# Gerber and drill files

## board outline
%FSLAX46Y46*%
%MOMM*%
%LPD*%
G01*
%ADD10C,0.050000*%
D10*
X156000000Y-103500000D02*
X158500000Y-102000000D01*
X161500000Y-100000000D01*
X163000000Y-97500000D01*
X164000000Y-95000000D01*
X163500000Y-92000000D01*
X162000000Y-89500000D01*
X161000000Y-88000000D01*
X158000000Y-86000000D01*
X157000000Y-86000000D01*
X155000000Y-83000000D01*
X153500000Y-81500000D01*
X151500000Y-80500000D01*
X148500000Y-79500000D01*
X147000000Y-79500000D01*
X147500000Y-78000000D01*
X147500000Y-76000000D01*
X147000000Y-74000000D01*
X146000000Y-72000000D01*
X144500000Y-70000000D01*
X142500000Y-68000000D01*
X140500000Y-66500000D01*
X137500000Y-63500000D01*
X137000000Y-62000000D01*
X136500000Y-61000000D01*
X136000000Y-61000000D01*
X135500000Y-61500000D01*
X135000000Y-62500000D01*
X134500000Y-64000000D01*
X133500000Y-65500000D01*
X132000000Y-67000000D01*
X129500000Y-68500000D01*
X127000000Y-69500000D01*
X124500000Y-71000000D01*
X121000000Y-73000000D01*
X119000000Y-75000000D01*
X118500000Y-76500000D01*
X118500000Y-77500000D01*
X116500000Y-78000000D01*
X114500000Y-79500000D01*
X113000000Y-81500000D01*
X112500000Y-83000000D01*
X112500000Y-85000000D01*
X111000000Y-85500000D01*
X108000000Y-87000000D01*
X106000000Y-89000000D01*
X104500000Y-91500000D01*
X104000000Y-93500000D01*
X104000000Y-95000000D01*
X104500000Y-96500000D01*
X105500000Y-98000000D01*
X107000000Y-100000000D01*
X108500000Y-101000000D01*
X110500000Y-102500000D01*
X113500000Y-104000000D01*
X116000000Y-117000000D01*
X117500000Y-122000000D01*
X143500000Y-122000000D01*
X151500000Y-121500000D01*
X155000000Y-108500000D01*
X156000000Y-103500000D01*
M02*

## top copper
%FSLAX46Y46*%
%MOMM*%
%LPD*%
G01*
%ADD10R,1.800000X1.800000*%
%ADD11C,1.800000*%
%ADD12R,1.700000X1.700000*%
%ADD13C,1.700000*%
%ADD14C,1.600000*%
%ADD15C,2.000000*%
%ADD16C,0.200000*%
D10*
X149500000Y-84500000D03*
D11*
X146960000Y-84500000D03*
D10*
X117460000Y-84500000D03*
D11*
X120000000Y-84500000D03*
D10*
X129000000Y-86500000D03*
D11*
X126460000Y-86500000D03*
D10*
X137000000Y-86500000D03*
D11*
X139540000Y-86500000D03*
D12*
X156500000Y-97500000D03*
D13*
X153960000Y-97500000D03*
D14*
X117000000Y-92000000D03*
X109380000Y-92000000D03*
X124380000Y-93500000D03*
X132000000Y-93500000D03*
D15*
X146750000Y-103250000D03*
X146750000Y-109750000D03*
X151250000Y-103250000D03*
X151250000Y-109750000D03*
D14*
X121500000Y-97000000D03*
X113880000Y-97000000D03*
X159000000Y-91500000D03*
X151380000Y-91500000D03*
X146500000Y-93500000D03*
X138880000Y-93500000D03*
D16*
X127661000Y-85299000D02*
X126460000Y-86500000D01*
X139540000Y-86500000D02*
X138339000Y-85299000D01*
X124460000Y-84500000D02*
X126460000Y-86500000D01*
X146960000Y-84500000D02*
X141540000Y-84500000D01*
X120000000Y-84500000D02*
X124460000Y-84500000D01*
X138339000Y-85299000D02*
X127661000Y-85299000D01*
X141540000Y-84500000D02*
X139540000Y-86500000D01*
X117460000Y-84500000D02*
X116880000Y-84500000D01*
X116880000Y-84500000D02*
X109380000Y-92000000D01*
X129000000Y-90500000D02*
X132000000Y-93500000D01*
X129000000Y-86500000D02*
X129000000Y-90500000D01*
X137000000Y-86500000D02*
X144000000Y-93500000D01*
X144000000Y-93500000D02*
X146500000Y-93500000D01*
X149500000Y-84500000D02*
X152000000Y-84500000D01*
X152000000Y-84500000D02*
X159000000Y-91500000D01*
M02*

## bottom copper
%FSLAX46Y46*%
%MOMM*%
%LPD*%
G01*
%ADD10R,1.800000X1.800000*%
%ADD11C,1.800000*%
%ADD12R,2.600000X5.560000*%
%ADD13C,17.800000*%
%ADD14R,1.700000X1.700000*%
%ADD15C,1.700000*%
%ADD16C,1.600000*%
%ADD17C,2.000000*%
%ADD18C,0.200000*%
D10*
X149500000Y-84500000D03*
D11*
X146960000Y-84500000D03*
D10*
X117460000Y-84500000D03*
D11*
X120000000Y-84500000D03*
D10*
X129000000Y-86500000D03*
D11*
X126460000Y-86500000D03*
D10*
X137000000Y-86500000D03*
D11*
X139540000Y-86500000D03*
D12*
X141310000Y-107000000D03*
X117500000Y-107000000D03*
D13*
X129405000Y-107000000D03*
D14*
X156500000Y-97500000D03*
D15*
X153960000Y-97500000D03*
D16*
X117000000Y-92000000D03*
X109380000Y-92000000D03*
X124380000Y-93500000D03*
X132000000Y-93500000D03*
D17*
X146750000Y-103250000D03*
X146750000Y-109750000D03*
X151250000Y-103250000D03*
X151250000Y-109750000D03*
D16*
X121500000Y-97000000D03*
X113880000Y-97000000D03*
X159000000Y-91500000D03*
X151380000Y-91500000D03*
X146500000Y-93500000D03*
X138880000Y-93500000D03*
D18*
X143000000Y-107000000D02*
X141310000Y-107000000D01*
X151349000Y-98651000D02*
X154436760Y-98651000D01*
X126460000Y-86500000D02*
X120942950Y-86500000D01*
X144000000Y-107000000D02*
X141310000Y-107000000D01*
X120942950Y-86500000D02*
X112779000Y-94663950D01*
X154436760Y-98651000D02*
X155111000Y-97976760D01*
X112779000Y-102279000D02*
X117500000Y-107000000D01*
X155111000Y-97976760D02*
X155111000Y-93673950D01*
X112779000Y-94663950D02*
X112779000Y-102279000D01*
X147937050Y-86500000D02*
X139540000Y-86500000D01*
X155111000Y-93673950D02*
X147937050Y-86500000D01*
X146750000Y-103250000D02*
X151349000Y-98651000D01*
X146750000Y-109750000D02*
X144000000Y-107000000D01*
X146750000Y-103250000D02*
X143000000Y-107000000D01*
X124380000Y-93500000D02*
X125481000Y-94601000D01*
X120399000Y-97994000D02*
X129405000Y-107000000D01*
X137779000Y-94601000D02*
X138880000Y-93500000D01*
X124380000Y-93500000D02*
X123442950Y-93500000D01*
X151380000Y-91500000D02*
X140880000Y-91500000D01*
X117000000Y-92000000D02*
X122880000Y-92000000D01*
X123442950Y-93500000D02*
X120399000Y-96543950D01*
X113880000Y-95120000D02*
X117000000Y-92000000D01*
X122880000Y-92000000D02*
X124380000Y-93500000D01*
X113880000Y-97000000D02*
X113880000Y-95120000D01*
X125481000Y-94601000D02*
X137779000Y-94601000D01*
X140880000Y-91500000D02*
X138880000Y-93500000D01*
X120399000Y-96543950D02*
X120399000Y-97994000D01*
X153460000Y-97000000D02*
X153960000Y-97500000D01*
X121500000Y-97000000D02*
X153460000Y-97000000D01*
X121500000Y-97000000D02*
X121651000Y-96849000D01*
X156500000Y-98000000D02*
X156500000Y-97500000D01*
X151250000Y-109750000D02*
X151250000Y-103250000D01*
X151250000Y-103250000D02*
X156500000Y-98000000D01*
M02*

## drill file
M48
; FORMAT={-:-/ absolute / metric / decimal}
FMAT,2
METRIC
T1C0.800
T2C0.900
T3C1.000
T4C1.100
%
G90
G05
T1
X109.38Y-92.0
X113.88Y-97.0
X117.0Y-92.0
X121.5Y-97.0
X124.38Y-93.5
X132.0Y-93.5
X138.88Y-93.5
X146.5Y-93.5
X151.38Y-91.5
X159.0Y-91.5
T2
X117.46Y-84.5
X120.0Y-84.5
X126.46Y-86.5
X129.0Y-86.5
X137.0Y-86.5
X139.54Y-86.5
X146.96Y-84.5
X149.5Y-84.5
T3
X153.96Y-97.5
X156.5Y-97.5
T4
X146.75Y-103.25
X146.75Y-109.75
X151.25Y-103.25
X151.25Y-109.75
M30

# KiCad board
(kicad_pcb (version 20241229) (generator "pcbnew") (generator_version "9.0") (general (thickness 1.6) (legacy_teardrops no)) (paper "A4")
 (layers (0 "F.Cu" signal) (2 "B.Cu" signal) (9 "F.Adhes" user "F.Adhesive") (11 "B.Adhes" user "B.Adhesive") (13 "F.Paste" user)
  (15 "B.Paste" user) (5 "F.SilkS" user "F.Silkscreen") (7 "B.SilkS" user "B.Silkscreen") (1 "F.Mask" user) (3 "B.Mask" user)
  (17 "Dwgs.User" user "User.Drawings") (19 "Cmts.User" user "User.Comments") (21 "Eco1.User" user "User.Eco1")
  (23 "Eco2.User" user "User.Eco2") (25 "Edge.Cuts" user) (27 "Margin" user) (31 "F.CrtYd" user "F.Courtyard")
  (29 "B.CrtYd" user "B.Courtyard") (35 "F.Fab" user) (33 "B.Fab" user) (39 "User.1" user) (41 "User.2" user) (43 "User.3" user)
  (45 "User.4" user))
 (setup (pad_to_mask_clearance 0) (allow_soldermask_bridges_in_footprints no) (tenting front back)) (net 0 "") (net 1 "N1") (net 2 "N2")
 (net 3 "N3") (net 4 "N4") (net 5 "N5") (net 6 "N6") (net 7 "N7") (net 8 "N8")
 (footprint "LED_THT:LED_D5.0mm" (layer "F.Cu") (at 149.5 84.5 180)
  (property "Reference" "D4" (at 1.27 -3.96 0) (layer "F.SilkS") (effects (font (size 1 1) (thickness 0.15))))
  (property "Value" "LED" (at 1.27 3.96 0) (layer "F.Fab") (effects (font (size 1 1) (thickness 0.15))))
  (pad "1" thru_hole rect (at 0 0 180) (size 1.8 1.8) (drill 0.9) (layers "*.Cu" "*.Mask") (remove_unused_layers no) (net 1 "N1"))
  (pad "2" thru_hole circle (at 2.54 0 180) (size 1.8 1.8) (drill 0.9) (layers "*.Cu" "*.Mask") (remove_unused_layers no) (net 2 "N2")))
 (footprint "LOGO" (layer "F.Cu") (at 134.5 112)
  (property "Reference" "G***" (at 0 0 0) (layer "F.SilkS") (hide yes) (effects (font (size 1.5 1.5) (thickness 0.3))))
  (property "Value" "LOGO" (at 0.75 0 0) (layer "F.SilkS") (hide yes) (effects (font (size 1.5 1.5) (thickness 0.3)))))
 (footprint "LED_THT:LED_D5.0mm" (layer "F.Cu") (at 117.46 84.5)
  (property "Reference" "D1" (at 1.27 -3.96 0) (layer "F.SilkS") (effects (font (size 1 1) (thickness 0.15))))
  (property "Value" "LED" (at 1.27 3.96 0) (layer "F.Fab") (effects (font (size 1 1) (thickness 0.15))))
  (pad "1" thru_hole rect (at 0 0) (size 1.8 1.8) (drill 0.9) (layers "*.Cu" "*.Mask") (remove_unused_layers no) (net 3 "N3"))
  (pad "2" thru_hole circle (at 2.54 0) (size 1.8 1.8) (drill 0.9) (layers "*.Cu" "*.Mask") (remove_unused_layers no) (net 2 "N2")))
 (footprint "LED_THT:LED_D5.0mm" (layer "F.Cu") (at 129 86.5 180)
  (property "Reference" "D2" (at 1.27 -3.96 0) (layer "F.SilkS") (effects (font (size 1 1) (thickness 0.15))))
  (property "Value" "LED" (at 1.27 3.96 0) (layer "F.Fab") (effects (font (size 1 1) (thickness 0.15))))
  (pad "1" thru_hole rect (at 0 0 180) (size 1.8 1.8) (drill 0.9) (layers "*.Cu" "*.Mask") (remove_unused_layers no) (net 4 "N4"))
  (pad "2" thru_hole circle (at 2.54 0 180) (size 1.8 1.8) (drill 0.9) (layers "*.Cu" "*.Mask") (remove_unused_layers no) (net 2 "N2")))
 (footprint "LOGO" (layer "F.Cu") (at 133 73.5)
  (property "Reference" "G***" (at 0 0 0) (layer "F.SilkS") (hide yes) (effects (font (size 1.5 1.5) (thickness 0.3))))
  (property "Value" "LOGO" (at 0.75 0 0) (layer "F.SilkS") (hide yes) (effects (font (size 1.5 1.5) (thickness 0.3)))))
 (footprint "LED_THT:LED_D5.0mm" (layer "F.Cu") (at 137 86.5)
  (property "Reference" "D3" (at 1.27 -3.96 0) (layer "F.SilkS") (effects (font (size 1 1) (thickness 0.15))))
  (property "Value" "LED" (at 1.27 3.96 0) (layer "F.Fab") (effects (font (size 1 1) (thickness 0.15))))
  (pad "1" thru_hole rect (at 0 0) (size 1.8 1.8) (drill 0.9) (layers "*.Cu" "*.Mask") (remove_unused_layers no) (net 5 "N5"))
  (pad "2" thru_hole circle (at 2.54 0) (size 1.8 1.8) (drill 0.9) (layers "*.Cu" "*.Mask") (remove_unused_layers no) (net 2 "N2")))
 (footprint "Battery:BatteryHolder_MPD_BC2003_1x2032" (layer "B.Cu") (at 129.405 107 180)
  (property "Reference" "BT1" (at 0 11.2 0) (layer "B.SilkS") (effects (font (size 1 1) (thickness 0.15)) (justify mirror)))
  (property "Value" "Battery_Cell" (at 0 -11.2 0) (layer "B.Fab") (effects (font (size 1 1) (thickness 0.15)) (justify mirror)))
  (pad "1" smd rect (at -11.905 0 180) (size 2.6 5.56) (layers "B.Cu" "B.Mask" "B.Paste") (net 2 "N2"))
  (pad "1" smd rect (at 11.905 0 180) (size 2.6 5.56) (layers "B.Cu" "B.Mask" "B.Paste") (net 2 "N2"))
  (pad "2" smd circle (at 0 0 180) (size 17.8 17.8) (layers "B.Cu" "B.Mask") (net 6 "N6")))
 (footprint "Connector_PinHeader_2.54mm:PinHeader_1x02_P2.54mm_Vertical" (layer "B.Cu") (at 156.5 97.5 90)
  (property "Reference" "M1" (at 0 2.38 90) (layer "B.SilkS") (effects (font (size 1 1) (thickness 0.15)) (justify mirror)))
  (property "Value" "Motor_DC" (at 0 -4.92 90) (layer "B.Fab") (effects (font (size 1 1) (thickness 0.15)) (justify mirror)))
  (pad "1" thru_hole rect (at 0 0 90) (size 1.7 1.7) (drill 1) (layers "*.Cu" "*.Mask") (remove_unused_layers no) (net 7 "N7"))
  (pad "2" thru_hole circle (at 0 -2.54 90) (size 1.7 1.7) (drill 1) (layers "*.Cu" "*.Mask") (remove_unused_layers no) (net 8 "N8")))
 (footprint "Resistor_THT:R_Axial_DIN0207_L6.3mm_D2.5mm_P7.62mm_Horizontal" (layer "B.Cu") (at 117 92 180)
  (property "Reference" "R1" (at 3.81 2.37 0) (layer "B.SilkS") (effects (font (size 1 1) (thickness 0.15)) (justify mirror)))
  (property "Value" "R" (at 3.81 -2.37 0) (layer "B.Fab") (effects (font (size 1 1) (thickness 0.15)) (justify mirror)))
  (pad "1" thru_hole circle (at 0 0 180) (size 1.6 1.6) (drill 0.8) (layers "*.Cu" "*.Mask") (remove_unused_layers no) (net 6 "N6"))
  (pad "2" thru_hole circle (at 7.62 0 180) (size 1.6 1.6) (drill 0.8) (layers "*.Cu" "*.Mask") (remove_unused_layers no) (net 3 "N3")))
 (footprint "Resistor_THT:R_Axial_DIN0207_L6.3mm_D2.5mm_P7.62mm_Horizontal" (layer "B.Cu") (at 124.38 93.5)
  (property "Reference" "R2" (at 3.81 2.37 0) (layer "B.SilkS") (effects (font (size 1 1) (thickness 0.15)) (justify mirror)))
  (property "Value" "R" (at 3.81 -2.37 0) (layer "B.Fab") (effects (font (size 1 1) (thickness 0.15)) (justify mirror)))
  (pad "1" thru_hole circle (at 0 0) (size 1.6 1.6) (drill 0.8) (layers "*.Cu" "*.Mask") (remove_unused_layers no) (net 6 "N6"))
  (pad "2" thru_hole circle (at 7.62 0) (size 1.6 1.6) (drill 0.8) (layers "*.Cu" "*.Mask") (remove_unused_layers no) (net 4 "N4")))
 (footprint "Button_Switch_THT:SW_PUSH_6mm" (layer "B.Cu") (at 146.75 103.25 -90)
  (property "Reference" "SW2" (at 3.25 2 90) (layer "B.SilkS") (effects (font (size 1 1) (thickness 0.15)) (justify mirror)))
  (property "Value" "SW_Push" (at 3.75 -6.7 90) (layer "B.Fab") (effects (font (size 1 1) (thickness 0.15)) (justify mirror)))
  (pad "1" thru_hole circle (at 0 0 180) (size 2 2) (drill 1.1) (layers "*.Cu" "*.Mask") (remove_unused_layers no) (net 2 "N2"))
  (pad "1" thru_hole circle (at 6.5 0 180) (size 2 2) (drill 1.1) (layers "*.Cu" "*.Mask") (remove_unused_layers no) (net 2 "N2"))
  (pad "2" thru_hole circle (at 0 -4.5 180) (size 2 2) (drill 1.1) (layers "*.Cu" "*.Mask") (remove_unused_layers no) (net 7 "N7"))
  (pad "2" thru_hole circle (at 6.5 -4.5 180) (size 2 2) (drill 1.1) (layers "*.Cu" "*.Mask") (remove_unused_layers no) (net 7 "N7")))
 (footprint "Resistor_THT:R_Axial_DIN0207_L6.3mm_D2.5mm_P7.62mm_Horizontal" (layer "B.Cu") (at 121.5 97 180)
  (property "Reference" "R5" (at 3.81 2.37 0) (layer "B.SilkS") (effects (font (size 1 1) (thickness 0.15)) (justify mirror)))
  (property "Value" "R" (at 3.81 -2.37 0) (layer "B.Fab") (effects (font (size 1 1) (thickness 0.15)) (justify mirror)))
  (pad "1" thru_hole circle (at 0 0 180) (size 1.6 1.6) (drill 0.8) (layers "*.Cu" "*.Mask") (remove_unused_layers no) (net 8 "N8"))
  (pad "2" thru_hole circle (at 7.62 0 180) (size 1.6 1.6) (drill 0.8) (layers "*.Cu" "*.Mask") (remove_unused_layers no) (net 6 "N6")))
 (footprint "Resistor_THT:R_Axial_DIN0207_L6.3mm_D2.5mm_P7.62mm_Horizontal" (layer "B.Cu") (at 159 91.5 180)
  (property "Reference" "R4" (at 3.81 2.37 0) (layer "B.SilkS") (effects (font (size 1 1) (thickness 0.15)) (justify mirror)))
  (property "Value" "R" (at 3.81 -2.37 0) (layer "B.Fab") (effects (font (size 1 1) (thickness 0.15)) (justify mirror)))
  (pad "1" thru_hole circle (at 0 0 180) (size 1.6 1.6) (drill 0.8) (layers "*.Cu" "*.Mask") (remove_unused_layers no) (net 1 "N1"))
  (pad "2" thru_hole circle (at 7.62 0 180) (size 1.6 1.6) (drill 0.8) (layers "*.Cu" "*.Mask") (remove_unused_layers no) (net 6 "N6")))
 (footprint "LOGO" (layer "B.Cu") (at 144 115 180)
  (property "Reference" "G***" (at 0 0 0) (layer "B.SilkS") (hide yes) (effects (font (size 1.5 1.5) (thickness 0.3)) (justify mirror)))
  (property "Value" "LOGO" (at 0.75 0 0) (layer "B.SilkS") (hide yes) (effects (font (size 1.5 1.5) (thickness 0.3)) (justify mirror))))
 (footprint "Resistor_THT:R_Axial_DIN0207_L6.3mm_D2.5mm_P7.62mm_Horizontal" (layer "B.Cu") (at 146.5 93.5 180)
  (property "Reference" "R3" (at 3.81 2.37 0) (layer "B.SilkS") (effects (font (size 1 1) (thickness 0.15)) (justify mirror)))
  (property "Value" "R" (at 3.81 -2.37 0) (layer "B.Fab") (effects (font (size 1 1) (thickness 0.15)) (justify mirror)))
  (pad "1" thru_hole circle (at 0 0 180) (size 1.6 1.6) (drill 0.8) (layers "*.Cu" "*.Mask") (remove_unused_layers no) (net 5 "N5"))
  (pad "2" thru_hole circle (at 7.62 0 180) (size 1.6 1.6) (drill 0.8) (layers "*.Cu" "*.Mask") (remove_unused_layers no) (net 6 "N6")))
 (gr_poly
  (pts (xy 156 103.5) (xy 158.5 102) (xy 161.5 100) (xy 163 97.5) (xy 164 95) (xy 163.5 92) (xy 162 89.5) (xy 161 88) (xy 158 86)
   (xy 157 86) (xy 155 83) (xy 153.5 81.5) (xy 151.5 80.5) (xy 148.5 79.5) (xy 147 79.5) (xy 147.5 78) (xy 147.5 76) (xy 147 74) (xy 146 72)
   (xy 144.5 70) (xy 142.5 68) (xy 140.5 66.5) (xy 137.5 63.5) (xy 137 62) (xy 136.5 61) (xy 136 61) (xy 135.5 61.5) (xy 135 62.5)
   (xy 134.5 64) (xy 133.5 65.5) (xy 132 67) (xy 129.5 68.5) (xy 127 69.5) (xy 124.5 71) (xy 121 73) (xy 119 75) (xy 118.5 76.5)
   (xy 118.5 77.5) (xy 116.5 78) (xy 114.5 79.5) (xy 113 81.5) (xy 112.5 83) (xy 112.5 85) (xy 111 85.5) (xy 108 87) (xy 106 89)
   (xy 104.5 91.5) (xy 104 93.5) (xy 104 95) (xy 104.5 96.5) (xy 105.5 98) (xy 107 100) (xy 108.5 101) (xy 110.5 102.5) (xy 113.5 104)
   (xy 116 117) (xy 117.5 122) (xy 143.5 122) (xy 151.5 121.5) (xy 155 108.5))
  (stroke (width 0.05) (type solid)) (fill no) (layer "Edge.Cuts"))
 (segment (start 127.661 85.299) (end 126.46 86.5) (width 0.2) (layer "F.Cu") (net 2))
 (segment (start 139.54 86.5) (end 138.339 85.299) (width 0.2) (layer "F.Cu") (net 2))
 (segment (start 124.46 84.5) (end 126.46 86.5) (width 0.2) (layer "F.Cu") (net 2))
 (segment (start 146.96 84.5) (end 141.54 84.5) (width 0.2) (layer "F.Cu") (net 2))
 (segment (start 120 84.5) (end 124.46 84.5) (width 0.2) (layer "F.Cu") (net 2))
 (segment (start 138.339 85.299) (end 127.661 85.299) (width 0.2) (layer "F.Cu") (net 2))
 (segment (start 141.54 84.5) (end 139.54 86.5) (width 0.2) (layer "F.Cu") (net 2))
 (segment (start 143 107) (end 141.31 107) (width 0.2) (layer "B.Cu") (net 2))
 (segment (start 151.349 98.651) (end 154.43676 98.651) (width 0.2) (layer "B.Cu") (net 2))
 (segment (start 126.46 86.5) (end 120.94295 86.5) (width 0.2) (layer "B.Cu") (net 2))
 (segment (start 144 107) (end 141.31 107) (width 0.2) (layer "B.Cu") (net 2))
 (segment (start 120.94295 86.5) (end 112.779 94.66395) (width 0.2) (layer "B.Cu") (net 2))
 (segment (start 154.43676 98.651) (end 155.111 97.97676) (width 0.2) (layer "B.Cu") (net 2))
 (segment (start 112.779 102.279) (end 117.5 107) (width 0.2) (layer "B.Cu") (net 2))
 (segment (start 155.111 97.97676) (end 155.111 93.67395) (width 0.2) (layer "B.Cu") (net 2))
 (segment (start 112.779 94.66395) (end 112.779 102.279) (width 0.2) (layer "B.Cu") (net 2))
 (segment (start 147.93705 86.5) (end 139.54 86.5) (width 0.2) (layer "B.Cu") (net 2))
 (segment (start 155.111 93.67395) (end 147.93705 86.5) (width 0.2) (layer "B.Cu") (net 2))
 (segment (start 146.75 103.25) (end 151.349 98.651) (width 0.2) (layer "B.Cu") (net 2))
 (segment (start 146.75 109.75) (end 144 107) (width 0.2) (layer "B.Cu") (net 2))
 (segment (start 146.75 103.25) (end 143 107) (width 0.2) (layer "B.Cu") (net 2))
 (segment (start 124.38 93.5) (end 125.481 94.601) (width 0.2) (layer "B.Cu") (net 6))
 (segment (start 120.399 97.994) (end 129.405 107) (width 0.2) (layer "B.Cu") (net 6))
 (segment (start 137.779 94.601) (end 138.88 93.5) (width 0.2) (layer "B.Cu") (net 6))
 (segment (start 124.38 93.5) (end 123.44295 93.5) (width 0.2) (layer "B.Cu") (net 6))
 (segment (start 151.38 91.5) (end 140.88 91.5) (width 0.2) (layer "B.Cu") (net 6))
 (segment (start 117 92) (end 122.88 92) (width 0.2) (layer "B.Cu") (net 6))
 (segment (start 123.44295 93.5) (end 120.399 96.54395) (width 0.2) (layer "B.Cu") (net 6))
 (segment (start 113.88 95.12) (end 117 92) (width 0.2) (layer "B.Cu") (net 6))
 (segment (start 122.88 92) (end 124.38 93.5) (width 0.2) (layer "B.Cu") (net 6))
 (segment (start 113.88 97) (end 113.88 95.12) (width 0.2) (layer "B.Cu") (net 6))
 (segment (start 125.481 94.601) (end 137.779 94.601) (width 0.2) (layer "B.Cu") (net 6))
 (segment (start 140.88 91.5) (end 138.88 93.5) (width 0.2) (layer "B.Cu") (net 6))
 (segment (start 120.399 96.54395) (end 120.399 97.994) (width 0.2) (layer "B.Cu") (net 6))
 (segment (start 117.46 84.5) (end 116.88 84.5) (width 0.2) (layer "F.Cu") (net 3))
 (segment (start 116.88 84.5) (end 109.38 92) (width 0.2) (layer "F.Cu") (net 3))
 (segment (start 129 90.5) (end 132 93.5) (width 0.2) (layer "F.Cu") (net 4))
 (segment (start 129 86.5) (end 129 90.5) (width 0.2) (layer "F.Cu") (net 4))
 (segment (start 137 86.5) (end 144 93.5) (width 0.2) (layer "F.Cu") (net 5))
 (segment (start 144 93.5) (end 146.5 93.5) (width 0.2) (layer "F.Cu") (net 5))
 (segment (start 149.5 84.5) (end 152 84.5) (width 0.2) (layer "F.Cu") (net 1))
 (segment (start 152 84.5) (end 159 91.5) (width 0.2) (layer "F.Cu") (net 1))
 (segment (start 153.46 97) (end 153.96 97.5) (width 0.2) (layer "B.Cu") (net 8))
 (segment (start 121.5 97) (end 153.46 97) (width 0.2) (layer "B.Cu") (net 8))
 (segment (start 121.5 97) (end 121.651 96.849) (width 0.2) (layer "B.Cu") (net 8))
 (segment (start 156.5 98) (end 156.5 97.5) (width 0.2) (layer "B.Cu") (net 7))
 (segment (start 151.25 109.75) (end 151.25 103.25) (width 0.2) (layer "B.Cu") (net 7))
 (segment (start 151.25 103.25) (end 156.5 98) (width 0.2) (layer "B.Cu") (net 7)))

